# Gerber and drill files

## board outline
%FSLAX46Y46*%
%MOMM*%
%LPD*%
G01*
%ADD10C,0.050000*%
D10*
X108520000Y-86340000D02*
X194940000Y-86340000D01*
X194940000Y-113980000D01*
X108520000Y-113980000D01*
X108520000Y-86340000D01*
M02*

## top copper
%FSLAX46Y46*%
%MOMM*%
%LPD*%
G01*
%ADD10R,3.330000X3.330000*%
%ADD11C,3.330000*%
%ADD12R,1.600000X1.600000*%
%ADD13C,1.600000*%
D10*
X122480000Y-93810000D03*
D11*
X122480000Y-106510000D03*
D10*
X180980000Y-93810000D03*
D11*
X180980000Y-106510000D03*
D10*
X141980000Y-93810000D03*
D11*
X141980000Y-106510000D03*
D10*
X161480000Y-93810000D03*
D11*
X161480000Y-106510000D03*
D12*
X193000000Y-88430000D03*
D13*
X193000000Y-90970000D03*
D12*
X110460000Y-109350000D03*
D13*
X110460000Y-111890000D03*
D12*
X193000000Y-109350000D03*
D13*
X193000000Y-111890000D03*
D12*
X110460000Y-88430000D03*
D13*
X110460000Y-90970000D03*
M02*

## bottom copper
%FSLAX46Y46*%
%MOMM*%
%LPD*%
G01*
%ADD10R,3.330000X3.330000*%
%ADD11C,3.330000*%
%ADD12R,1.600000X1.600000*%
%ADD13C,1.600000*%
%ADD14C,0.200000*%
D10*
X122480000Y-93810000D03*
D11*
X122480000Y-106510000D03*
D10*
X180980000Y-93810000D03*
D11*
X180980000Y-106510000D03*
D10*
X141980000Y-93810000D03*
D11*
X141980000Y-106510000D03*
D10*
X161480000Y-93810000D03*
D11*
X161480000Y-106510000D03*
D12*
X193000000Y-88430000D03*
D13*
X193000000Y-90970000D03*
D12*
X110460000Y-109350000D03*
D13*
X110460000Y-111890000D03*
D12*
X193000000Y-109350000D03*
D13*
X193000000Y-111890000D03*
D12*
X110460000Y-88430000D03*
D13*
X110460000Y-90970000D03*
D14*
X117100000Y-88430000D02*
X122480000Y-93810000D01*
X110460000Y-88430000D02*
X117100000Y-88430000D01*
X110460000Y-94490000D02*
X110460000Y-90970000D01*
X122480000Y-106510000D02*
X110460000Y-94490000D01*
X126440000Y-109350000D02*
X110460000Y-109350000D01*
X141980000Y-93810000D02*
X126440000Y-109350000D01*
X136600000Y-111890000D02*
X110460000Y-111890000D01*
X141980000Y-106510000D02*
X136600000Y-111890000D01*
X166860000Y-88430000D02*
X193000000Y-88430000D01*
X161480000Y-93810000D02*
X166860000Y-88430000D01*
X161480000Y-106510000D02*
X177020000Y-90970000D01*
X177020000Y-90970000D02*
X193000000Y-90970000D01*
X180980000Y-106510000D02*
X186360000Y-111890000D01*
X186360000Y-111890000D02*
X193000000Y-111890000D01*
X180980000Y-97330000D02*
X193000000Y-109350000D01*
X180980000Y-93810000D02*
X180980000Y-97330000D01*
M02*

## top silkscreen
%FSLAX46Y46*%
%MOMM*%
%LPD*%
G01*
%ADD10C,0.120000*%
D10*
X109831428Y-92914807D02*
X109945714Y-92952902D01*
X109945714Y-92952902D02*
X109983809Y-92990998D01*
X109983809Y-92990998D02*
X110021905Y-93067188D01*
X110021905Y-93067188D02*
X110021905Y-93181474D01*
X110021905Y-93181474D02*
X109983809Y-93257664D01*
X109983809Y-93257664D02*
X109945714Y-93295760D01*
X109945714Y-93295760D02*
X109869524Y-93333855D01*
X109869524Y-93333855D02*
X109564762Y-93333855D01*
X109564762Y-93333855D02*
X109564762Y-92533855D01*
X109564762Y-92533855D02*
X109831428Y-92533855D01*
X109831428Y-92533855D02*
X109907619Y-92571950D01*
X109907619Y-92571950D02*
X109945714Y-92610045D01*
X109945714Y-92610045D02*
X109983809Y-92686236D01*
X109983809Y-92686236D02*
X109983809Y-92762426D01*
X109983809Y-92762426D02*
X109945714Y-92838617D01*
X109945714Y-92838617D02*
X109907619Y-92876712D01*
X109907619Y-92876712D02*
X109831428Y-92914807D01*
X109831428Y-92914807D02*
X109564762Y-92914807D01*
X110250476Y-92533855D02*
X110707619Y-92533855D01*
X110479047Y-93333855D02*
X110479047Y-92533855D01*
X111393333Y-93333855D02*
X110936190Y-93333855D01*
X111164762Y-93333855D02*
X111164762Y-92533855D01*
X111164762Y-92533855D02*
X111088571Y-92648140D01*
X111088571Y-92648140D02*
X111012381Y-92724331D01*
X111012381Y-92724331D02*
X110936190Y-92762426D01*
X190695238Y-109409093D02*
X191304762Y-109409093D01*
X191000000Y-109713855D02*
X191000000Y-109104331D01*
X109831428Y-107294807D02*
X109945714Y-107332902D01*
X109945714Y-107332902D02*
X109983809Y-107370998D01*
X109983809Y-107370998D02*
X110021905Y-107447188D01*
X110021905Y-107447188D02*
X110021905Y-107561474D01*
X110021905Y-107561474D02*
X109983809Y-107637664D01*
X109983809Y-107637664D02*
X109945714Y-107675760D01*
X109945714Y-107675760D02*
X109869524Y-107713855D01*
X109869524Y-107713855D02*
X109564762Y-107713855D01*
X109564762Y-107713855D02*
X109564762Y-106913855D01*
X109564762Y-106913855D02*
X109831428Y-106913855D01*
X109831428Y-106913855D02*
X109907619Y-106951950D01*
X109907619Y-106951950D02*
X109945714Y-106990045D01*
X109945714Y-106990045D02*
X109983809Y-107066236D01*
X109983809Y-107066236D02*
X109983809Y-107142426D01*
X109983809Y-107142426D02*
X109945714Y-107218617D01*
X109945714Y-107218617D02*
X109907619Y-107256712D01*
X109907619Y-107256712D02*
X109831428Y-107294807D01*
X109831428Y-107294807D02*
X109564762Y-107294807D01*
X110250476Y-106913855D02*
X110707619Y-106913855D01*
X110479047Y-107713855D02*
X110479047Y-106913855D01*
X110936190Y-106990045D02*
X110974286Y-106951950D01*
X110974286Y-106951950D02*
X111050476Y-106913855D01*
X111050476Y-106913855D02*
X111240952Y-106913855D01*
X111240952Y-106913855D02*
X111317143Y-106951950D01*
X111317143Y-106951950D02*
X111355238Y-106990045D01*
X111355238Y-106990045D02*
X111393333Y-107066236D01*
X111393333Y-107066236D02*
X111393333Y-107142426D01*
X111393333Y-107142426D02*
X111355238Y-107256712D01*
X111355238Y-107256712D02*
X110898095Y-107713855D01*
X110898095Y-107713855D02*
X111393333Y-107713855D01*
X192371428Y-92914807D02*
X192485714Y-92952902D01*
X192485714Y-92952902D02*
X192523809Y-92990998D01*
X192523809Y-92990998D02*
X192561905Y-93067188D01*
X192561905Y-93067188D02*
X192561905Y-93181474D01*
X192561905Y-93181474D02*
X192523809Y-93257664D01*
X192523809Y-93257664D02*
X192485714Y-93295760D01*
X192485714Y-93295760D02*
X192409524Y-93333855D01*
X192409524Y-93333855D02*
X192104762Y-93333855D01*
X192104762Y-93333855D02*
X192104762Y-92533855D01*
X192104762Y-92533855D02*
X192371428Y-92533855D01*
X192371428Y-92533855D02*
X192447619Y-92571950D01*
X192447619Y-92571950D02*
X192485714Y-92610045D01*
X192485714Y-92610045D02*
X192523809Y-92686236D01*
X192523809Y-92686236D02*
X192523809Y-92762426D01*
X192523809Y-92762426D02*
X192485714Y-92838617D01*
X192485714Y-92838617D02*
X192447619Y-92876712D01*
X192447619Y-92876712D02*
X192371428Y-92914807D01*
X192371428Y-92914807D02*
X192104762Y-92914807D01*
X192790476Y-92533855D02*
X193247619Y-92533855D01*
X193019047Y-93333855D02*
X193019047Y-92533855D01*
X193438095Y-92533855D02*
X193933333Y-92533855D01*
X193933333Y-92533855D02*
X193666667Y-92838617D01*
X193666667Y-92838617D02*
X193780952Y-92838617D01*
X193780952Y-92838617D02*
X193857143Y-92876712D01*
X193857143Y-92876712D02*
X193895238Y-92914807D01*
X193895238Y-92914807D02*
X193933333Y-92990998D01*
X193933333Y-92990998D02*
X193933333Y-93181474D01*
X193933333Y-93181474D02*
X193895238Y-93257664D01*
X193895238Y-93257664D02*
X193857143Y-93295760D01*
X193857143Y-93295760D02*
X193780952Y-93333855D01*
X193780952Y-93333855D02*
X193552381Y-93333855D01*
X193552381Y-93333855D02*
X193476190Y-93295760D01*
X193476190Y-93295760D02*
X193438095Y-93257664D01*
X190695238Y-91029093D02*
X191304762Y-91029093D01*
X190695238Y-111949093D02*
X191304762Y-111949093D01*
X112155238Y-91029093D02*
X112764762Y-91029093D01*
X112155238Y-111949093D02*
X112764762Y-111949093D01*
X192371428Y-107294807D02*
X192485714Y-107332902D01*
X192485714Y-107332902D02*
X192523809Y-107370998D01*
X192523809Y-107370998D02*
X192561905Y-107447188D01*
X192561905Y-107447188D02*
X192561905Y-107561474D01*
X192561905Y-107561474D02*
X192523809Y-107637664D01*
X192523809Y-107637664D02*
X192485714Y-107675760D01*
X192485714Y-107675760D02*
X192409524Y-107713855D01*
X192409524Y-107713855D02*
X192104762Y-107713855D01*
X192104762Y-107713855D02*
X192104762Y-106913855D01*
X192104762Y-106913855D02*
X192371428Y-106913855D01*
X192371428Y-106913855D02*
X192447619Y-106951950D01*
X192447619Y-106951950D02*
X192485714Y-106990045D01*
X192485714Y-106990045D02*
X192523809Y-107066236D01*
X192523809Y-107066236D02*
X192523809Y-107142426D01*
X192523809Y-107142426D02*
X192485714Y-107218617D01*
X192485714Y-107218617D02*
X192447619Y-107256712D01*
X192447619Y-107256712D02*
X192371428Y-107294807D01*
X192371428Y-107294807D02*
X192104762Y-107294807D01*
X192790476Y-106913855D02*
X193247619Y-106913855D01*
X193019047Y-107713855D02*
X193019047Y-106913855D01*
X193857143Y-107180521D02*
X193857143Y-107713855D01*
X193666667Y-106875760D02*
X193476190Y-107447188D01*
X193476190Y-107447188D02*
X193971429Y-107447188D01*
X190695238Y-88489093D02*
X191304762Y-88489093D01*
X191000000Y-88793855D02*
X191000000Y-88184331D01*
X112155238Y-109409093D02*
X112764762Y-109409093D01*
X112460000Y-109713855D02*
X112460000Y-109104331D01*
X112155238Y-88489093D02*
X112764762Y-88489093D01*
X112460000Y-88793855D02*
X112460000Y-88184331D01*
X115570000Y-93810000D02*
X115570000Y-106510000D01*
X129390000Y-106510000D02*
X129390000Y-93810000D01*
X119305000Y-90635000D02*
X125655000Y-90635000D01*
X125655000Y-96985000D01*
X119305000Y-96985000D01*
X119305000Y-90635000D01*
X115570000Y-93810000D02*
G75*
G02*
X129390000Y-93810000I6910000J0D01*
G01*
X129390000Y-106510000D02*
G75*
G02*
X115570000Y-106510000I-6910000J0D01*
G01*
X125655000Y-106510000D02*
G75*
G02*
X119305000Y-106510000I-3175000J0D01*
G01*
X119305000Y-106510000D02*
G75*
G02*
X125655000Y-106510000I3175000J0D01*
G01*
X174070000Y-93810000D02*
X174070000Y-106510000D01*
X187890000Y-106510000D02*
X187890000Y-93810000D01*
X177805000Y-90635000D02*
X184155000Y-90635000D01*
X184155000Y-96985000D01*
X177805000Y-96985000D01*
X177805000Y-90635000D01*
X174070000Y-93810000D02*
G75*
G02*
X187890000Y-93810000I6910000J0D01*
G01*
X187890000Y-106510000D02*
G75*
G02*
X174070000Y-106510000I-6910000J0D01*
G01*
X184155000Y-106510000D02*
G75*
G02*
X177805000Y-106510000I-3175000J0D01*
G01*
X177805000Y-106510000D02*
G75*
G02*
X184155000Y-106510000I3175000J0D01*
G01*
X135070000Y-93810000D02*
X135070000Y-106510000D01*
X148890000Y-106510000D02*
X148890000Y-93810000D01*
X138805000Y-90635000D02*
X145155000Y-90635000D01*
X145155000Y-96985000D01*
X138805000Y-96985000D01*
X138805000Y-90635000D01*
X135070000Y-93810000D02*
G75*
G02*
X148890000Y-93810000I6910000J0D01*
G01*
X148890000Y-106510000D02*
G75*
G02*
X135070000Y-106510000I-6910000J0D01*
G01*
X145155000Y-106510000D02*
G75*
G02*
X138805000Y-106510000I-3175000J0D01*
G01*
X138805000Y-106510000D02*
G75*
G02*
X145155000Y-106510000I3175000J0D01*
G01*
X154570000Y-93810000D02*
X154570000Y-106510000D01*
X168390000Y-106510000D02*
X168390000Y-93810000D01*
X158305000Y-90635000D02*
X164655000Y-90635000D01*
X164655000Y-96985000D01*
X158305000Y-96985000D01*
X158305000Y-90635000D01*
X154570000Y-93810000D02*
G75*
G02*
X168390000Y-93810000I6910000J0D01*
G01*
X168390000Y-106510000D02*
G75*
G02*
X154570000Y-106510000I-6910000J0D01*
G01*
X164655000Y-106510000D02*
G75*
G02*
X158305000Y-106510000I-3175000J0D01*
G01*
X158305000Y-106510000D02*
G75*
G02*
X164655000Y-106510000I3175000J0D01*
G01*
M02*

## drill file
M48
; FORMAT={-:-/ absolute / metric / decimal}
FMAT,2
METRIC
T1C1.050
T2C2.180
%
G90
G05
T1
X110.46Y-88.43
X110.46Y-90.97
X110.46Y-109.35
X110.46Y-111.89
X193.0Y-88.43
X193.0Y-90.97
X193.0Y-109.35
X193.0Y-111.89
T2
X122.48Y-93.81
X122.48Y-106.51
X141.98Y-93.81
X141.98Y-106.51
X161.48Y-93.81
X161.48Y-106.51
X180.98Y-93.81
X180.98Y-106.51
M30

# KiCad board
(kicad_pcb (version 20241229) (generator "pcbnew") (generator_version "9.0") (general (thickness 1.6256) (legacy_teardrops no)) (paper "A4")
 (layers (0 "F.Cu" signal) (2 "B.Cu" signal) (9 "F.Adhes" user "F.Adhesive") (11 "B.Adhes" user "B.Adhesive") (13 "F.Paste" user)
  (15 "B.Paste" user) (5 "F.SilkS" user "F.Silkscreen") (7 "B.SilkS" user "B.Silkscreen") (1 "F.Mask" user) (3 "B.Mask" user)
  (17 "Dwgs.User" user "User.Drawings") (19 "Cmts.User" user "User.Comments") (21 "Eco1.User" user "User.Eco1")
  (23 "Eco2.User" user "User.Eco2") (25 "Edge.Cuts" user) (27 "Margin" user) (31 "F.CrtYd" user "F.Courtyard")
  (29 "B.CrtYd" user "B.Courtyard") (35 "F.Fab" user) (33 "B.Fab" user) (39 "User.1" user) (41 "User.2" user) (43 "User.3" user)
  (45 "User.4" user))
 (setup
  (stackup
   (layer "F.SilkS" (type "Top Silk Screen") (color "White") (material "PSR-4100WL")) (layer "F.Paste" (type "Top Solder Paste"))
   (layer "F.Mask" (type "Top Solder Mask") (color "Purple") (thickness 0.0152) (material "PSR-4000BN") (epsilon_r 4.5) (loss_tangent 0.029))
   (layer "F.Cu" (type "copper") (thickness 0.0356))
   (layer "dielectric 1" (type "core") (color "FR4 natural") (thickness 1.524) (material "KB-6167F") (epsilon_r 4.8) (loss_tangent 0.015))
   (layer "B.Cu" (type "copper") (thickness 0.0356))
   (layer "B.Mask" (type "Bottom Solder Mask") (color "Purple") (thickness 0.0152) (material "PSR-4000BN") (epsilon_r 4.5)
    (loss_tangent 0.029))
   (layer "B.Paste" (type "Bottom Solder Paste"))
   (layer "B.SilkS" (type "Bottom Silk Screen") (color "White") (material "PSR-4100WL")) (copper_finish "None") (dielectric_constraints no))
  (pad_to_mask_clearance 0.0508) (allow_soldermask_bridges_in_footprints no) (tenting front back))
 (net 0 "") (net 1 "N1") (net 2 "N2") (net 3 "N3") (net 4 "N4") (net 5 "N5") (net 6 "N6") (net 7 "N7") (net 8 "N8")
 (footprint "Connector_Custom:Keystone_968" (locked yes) (layer "F.Cu") (at 122.48 100.16 -90)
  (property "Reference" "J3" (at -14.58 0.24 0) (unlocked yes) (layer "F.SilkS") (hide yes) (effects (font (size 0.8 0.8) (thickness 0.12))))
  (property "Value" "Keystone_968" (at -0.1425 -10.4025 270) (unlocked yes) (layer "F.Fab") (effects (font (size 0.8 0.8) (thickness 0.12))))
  (fp_line (start -6.35 6.91) (end 6.35 6.91) (stroke (width 0.12) (type default)) (layer "F.SilkS"))
  (fp_line (start 6.35 -6.91) (end -6.35 -6.91) (stroke (width 0.12) (type default)) (layer "F.SilkS"))
  (fp_rect (start -9.525 -3.175) (end -3.175 3.175) (stroke (width 0.12) (type default)) (fill no) (layer "F.SilkS"))
  (fp_arc (start -6.35 6.91) (mid -13.26 0) (end -6.35 -6.91) (stroke (width 0.12) (type default)) (layer "F.SilkS"))
  (fp_arc (start 6.35 -6.91) (mid 13.26 0) (end 6.35 6.91) (stroke (width 0.12) (type default)) (layer "F.SilkS"))
  (fp_circle (center 6.35 0) (end 9.525 0) (stroke (width 0.12) (type default)) (fill no) (layer "F.SilkS"))
  (pad "1" thru_hole rect (at -6.35 0 270) (size 3.33 3.33) (drill 2.18) (layers "*.Cu" "*.Mask") (remove_unused_layers no) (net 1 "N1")
   (thermal_bridge_angle 45))
  (pad "2" thru_hole circle (at 6.35 0 270) (size 3.33 3.33) (drill 2.18) (layers "*.Cu" "*.Mask") (remove_unused_layers no) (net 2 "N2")))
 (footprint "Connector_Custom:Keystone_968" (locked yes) (layer "F.Cu") (at 180.98 100.16 -90)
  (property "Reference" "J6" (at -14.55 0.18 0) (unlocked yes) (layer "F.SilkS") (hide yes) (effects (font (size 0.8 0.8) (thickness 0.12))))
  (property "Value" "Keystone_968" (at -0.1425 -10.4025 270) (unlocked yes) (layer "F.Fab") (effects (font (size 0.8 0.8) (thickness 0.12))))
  (fp_line (start -6.35 6.91) (end 6.35 6.91) (stroke (width 0.12) (type default)) (layer "F.SilkS"))
  (fp_line (start 6.35 -6.91) (end -6.35 -6.91) (stroke (width 0.12) (type default)) (layer "F.SilkS"))
  (fp_rect (start -9.525 -3.175) (end -3.175 3.175) (stroke (width 0.12) (type default)) (fill no) (layer "F.SilkS"))
  (fp_arc (start -6.35 6.91) (mid -13.26 0) (end -6.35 -6.91) (stroke (width 0.12) (type default)) (layer "F.SilkS"))
  (fp_arc (start 6.35 -6.91) (mid 13.26 0) (end 6.35 6.91) (stroke (width 0.12) (type default)) (layer "F.SilkS"))
  (fp_circle (center 6.35 0) (end 9.525 0) (stroke (width 0.12) (type default)) (fill no) (layer "F.SilkS"))
  (pad "1" thru_hole rect (at -6.35 0 270) (size 3.33 3.33) (drill 2.18) (layers "*.Cu" "*.Mask") (remove_unused_layers no) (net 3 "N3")
   (thermal_bridge_angle 45))
  (pad "2" thru_hole circle (at 6.35 0 270) (size 3.33 3.33) (drill 2.18) (layers "*.Cu" "*.Mask") (remove_unused_layers no) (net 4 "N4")))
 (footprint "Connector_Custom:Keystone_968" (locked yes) (layer "F.Cu") (at 141.98 100.16 -90)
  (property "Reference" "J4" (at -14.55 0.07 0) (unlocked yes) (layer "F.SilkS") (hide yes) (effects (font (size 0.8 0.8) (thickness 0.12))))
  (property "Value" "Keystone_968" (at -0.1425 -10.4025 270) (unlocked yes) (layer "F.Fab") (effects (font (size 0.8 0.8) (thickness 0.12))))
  (fp_line (start -6.35 6.91) (end 6.35 6.91) (stroke (width 0.12) (type default)) (layer "F.SilkS"))
  (fp_line (start 6.35 -6.91) (end -6.35 -6.91) (stroke (width 0.12) (type default)) (layer "F.SilkS"))
  (fp_rect (start -9.525 -3.175) (end -3.175 3.175) (stroke (width 0.12) (type default)) (fill no) (layer "F.SilkS"))
  (fp_arc (start -6.35 6.91) (mid -13.26 0) (end -6.35 -6.91) (stroke (width 0.12) (type default)) (layer "F.SilkS"))
  (fp_arc (start 6.35 -6.91) (mid 13.26 0) (end 6.35 6.91) (stroke (width 0.12) (type default)) (layer "F.SilkS"))
  (fp_circle (center 6.35 0) (end 9.525 0) (stroke (width 0.12) (type default)) (fill no) (layer "F.SilkS"))
  (pad "1" thru_hole rect (at -6.35 0 270) (size 3.33 3.33) (drill 2.18) (layers "*.Cu" "*.Mask") (remove_unused_layers no) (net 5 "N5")
   (thermal_bridge_angle 45))
  (pad "2" thru_hole circle (at 6.35 0 270) (size 3.33 3.33) (drill 2.18) (layers "*.Cu" "*.Mask") (remove_unused_layers no) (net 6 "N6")))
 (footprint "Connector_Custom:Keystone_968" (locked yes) (layer "F.Cu") (at 161.48 100.16 -90)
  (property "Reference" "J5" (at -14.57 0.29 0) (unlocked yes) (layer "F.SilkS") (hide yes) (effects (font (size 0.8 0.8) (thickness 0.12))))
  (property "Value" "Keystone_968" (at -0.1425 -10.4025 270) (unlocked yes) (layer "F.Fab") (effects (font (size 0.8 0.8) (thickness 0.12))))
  (fp_line (start -6.35 6.91) (end 6.35 6.91) (stroke (width 0.12) (type default)) (layer "F.SilkS"))
  (fp_line (start 6.35 -6.91) (end -6.35 -6.91) (stroke (width 0.12) (type default)) (layer "F.SilkS"))
  (fp_rect (start -9.525 -3.175) (end -3.175 3.175) (stroke (width 0.12) (type default)) (fill no) (layer "F.SilkS"))
  (fp_arc (start -6.35 6.91) (mid -13.26 0) (end -6.35 -6.91) (stroke (width 0.12) (type default)) (layer "F.SilkS"))
  (fp_arc (start 6.35 -6.91) (mid 13.26 0) (end 6.35 6.91) (stroke (width 0.12) (type default)) (layer "F.SilkS"))
  (fp_circle (center 6.35 0) (end 9.525 0) (stroke (width 0.12) (type default)) (fill no) (layer "F.SilkS"))
  (pad "1" thru_hole rect (at -6.35 0 270) (size 3.33 3.33) (drill 2.18) (layers "*.Cu" "*.Mask") (remove_unused_layers no) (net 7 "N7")
   (thermal_bridge_angle 45))
  (pad "2" thru_hole circle (at 6.35 0 270) (size 3.33 3.33) (drill 2.18) (layers "*.Cu" "*.Mask") (remove_unused_layers no) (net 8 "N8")))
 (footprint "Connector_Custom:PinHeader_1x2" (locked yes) (layer "B.Cu") (at 193 89.7 180)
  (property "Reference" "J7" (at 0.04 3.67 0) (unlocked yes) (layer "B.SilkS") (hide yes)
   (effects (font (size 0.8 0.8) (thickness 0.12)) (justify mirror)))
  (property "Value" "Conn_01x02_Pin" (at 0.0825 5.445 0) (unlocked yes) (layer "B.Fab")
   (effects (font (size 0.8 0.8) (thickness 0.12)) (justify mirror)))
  (pad "1" thru_hole rect (at 0 1.27 180) (size 1.6 1.6) (drill 1.05) (layers "*.Cu" "*.Mask") (remove_unused_layers no) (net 7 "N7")
   (thermal_bridge_angle 45))
  (pad "2" thru_hole circle (at 0 -1.27 180) (size 1.6 1.6) (drill 1.05) (layers "*.Cu" "*.Mask") (remove_unused_layers no) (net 8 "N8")))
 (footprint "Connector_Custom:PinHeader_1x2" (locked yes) (layer "B.Cu") (at 110.46 110.62 180)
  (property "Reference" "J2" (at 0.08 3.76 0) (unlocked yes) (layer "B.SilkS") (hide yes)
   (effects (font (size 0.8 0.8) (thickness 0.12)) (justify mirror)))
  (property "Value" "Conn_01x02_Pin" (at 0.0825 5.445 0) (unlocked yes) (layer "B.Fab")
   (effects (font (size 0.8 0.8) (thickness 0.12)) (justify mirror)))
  (pad "1" thru_hole rect (at 0 1.27 180) (size 1.6 1.6) (drill 1.05) (layers "*.Cu" "*.Mask") (remove_unused_layers no) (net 5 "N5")
   (thermal_bridge_angle 45))
  (pad "2" thru_hole circle (at 0 -1.27 180) (size 1.6 1.6) (drill 1.05) (layers "*.Cu" "*.Mask") (remove_unused_layers no) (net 6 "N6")))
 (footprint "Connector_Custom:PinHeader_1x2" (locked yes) (layer "B.Cu") (at 193 110.62 180)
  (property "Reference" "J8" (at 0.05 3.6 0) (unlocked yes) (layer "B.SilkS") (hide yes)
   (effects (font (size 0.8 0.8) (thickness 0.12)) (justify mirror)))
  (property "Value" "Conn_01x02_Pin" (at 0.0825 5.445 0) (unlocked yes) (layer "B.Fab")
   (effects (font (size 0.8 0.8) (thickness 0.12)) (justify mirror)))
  (pad "1" thru_hole rect (at 0 1.27 180) (size 1.6 1.6) (drill 1.05) (layers "*.Cu" "*.Mask") (remove_unused_layers no) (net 3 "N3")
   (thermal_bridge_angle 45))
  (pad "2" thru_hole circle (at 0 -1.27 180) (size 1.6 1.6) (drill 1.05) (layers "*.Cu" "*.Mask") (remove_unused_layers no) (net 4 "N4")))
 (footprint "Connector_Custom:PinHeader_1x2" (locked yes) (layer "B.Cu") (at 110.46 89.7 180)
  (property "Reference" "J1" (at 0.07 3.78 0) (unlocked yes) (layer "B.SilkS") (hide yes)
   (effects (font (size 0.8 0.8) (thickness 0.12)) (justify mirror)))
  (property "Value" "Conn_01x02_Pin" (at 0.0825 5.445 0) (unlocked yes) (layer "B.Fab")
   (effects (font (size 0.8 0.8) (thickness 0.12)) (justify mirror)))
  (pad "1" thru_hole rect (at 0 1.27 180) (size 1.6 1.6) (drill 1.05) (layers "*.Cu" "*.Mask") (remove_unused_layers no) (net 1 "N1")
   (thermal_bridge_angle 45))
  (pad "2" thru_hole circle (at 0 -1.27 180) (size 1.6 1.6) (drill 1.05) (layers "*.Cu" "*.Mask") (remove_unused_layers no) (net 2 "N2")))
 (gr_rect (start 108.52 86.34) (end 194.94 113.98) (stroke (width 0.05) (type default)) (fill no) (layer "Edge.Cuts"))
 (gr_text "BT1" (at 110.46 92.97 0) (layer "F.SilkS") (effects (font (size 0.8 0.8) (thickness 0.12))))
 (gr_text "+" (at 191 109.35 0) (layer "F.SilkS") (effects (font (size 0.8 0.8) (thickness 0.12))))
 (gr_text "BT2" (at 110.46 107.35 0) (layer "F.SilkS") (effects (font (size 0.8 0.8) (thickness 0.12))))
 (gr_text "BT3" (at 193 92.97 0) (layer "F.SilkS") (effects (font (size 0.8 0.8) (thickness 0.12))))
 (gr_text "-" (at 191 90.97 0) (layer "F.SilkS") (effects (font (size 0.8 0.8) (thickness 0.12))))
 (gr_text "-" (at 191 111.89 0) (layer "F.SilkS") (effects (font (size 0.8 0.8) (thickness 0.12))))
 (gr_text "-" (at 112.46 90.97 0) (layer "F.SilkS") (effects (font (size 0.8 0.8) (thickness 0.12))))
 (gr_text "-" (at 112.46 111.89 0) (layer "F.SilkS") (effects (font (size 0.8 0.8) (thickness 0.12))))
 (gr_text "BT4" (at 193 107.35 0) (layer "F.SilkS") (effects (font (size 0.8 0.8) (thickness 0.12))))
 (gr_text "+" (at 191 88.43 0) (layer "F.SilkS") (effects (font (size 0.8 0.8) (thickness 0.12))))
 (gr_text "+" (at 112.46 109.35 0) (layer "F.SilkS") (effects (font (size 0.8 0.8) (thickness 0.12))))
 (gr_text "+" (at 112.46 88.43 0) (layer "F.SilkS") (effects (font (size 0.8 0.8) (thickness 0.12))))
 (segment (start 117.1 88.43) (end 122.48 93.81) (width 0.2) (layer "B.Cu") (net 1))
 (segment (start 110.46 88.43) (end 117.1 88.43) (width 0.2) (layer "B.Cu") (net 1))
 (segment (start 110.46 94.49) (end 110.46 90.97) (width 0.2) (layer "B.Cu") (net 2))
 (segment (start 122.48 106.51) (end 110.46 94.49) (width 0.2) (layer "B.Cu") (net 2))
 (segment (start 126.44 109.35) (end 110.46 109.35) (width 0.2) (layer "B.Cu") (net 5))
 (segment (start 141.98 93.81) (end 126.44 109.35) (width 0.2) (layer "B.Cu") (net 5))
 (segment (start 136.6 111.89) (end 110.46 111.89) (width 0.2) (layer "B.Cu") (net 6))
 (segment (start 141.98 106.51) (end 136.6 111.89) (width 0.2) (layer "B.Cu") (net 6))
 (segment (start 166.86 88.43) (end 193 88.43) (width 0.2) (layer "B.Cu") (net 7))
 (segment (start 161.48 93.81) (end 166.86 88.43) (width 0.2) (layer "B.Cu") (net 7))
 (segment (start 161.48 106.51) (end 177.02 90.97) (width 0.2) (layer "B.Cu") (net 8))
 (segment (start 177.02 90.97) (end 193 90.97) (width 0.2) (layer "B.Cu") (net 8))
 (segment (start 180.98 106.51) (end 186.36 111.89) (width 0.2) (layer "B.Cu") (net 4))
 (segment (start 186.36 111.89) (end 193 111.89) (width 0.2) (layer "B.Cu") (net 4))
 (segment (start 180.98 97.33) (end 193 109.35) (width 0.2) (layer "B.Cu") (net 3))
 (segment (start 180.98 93.81) (end 180.98 97.33) (width 0.2) (layer "B.Cu") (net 3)))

